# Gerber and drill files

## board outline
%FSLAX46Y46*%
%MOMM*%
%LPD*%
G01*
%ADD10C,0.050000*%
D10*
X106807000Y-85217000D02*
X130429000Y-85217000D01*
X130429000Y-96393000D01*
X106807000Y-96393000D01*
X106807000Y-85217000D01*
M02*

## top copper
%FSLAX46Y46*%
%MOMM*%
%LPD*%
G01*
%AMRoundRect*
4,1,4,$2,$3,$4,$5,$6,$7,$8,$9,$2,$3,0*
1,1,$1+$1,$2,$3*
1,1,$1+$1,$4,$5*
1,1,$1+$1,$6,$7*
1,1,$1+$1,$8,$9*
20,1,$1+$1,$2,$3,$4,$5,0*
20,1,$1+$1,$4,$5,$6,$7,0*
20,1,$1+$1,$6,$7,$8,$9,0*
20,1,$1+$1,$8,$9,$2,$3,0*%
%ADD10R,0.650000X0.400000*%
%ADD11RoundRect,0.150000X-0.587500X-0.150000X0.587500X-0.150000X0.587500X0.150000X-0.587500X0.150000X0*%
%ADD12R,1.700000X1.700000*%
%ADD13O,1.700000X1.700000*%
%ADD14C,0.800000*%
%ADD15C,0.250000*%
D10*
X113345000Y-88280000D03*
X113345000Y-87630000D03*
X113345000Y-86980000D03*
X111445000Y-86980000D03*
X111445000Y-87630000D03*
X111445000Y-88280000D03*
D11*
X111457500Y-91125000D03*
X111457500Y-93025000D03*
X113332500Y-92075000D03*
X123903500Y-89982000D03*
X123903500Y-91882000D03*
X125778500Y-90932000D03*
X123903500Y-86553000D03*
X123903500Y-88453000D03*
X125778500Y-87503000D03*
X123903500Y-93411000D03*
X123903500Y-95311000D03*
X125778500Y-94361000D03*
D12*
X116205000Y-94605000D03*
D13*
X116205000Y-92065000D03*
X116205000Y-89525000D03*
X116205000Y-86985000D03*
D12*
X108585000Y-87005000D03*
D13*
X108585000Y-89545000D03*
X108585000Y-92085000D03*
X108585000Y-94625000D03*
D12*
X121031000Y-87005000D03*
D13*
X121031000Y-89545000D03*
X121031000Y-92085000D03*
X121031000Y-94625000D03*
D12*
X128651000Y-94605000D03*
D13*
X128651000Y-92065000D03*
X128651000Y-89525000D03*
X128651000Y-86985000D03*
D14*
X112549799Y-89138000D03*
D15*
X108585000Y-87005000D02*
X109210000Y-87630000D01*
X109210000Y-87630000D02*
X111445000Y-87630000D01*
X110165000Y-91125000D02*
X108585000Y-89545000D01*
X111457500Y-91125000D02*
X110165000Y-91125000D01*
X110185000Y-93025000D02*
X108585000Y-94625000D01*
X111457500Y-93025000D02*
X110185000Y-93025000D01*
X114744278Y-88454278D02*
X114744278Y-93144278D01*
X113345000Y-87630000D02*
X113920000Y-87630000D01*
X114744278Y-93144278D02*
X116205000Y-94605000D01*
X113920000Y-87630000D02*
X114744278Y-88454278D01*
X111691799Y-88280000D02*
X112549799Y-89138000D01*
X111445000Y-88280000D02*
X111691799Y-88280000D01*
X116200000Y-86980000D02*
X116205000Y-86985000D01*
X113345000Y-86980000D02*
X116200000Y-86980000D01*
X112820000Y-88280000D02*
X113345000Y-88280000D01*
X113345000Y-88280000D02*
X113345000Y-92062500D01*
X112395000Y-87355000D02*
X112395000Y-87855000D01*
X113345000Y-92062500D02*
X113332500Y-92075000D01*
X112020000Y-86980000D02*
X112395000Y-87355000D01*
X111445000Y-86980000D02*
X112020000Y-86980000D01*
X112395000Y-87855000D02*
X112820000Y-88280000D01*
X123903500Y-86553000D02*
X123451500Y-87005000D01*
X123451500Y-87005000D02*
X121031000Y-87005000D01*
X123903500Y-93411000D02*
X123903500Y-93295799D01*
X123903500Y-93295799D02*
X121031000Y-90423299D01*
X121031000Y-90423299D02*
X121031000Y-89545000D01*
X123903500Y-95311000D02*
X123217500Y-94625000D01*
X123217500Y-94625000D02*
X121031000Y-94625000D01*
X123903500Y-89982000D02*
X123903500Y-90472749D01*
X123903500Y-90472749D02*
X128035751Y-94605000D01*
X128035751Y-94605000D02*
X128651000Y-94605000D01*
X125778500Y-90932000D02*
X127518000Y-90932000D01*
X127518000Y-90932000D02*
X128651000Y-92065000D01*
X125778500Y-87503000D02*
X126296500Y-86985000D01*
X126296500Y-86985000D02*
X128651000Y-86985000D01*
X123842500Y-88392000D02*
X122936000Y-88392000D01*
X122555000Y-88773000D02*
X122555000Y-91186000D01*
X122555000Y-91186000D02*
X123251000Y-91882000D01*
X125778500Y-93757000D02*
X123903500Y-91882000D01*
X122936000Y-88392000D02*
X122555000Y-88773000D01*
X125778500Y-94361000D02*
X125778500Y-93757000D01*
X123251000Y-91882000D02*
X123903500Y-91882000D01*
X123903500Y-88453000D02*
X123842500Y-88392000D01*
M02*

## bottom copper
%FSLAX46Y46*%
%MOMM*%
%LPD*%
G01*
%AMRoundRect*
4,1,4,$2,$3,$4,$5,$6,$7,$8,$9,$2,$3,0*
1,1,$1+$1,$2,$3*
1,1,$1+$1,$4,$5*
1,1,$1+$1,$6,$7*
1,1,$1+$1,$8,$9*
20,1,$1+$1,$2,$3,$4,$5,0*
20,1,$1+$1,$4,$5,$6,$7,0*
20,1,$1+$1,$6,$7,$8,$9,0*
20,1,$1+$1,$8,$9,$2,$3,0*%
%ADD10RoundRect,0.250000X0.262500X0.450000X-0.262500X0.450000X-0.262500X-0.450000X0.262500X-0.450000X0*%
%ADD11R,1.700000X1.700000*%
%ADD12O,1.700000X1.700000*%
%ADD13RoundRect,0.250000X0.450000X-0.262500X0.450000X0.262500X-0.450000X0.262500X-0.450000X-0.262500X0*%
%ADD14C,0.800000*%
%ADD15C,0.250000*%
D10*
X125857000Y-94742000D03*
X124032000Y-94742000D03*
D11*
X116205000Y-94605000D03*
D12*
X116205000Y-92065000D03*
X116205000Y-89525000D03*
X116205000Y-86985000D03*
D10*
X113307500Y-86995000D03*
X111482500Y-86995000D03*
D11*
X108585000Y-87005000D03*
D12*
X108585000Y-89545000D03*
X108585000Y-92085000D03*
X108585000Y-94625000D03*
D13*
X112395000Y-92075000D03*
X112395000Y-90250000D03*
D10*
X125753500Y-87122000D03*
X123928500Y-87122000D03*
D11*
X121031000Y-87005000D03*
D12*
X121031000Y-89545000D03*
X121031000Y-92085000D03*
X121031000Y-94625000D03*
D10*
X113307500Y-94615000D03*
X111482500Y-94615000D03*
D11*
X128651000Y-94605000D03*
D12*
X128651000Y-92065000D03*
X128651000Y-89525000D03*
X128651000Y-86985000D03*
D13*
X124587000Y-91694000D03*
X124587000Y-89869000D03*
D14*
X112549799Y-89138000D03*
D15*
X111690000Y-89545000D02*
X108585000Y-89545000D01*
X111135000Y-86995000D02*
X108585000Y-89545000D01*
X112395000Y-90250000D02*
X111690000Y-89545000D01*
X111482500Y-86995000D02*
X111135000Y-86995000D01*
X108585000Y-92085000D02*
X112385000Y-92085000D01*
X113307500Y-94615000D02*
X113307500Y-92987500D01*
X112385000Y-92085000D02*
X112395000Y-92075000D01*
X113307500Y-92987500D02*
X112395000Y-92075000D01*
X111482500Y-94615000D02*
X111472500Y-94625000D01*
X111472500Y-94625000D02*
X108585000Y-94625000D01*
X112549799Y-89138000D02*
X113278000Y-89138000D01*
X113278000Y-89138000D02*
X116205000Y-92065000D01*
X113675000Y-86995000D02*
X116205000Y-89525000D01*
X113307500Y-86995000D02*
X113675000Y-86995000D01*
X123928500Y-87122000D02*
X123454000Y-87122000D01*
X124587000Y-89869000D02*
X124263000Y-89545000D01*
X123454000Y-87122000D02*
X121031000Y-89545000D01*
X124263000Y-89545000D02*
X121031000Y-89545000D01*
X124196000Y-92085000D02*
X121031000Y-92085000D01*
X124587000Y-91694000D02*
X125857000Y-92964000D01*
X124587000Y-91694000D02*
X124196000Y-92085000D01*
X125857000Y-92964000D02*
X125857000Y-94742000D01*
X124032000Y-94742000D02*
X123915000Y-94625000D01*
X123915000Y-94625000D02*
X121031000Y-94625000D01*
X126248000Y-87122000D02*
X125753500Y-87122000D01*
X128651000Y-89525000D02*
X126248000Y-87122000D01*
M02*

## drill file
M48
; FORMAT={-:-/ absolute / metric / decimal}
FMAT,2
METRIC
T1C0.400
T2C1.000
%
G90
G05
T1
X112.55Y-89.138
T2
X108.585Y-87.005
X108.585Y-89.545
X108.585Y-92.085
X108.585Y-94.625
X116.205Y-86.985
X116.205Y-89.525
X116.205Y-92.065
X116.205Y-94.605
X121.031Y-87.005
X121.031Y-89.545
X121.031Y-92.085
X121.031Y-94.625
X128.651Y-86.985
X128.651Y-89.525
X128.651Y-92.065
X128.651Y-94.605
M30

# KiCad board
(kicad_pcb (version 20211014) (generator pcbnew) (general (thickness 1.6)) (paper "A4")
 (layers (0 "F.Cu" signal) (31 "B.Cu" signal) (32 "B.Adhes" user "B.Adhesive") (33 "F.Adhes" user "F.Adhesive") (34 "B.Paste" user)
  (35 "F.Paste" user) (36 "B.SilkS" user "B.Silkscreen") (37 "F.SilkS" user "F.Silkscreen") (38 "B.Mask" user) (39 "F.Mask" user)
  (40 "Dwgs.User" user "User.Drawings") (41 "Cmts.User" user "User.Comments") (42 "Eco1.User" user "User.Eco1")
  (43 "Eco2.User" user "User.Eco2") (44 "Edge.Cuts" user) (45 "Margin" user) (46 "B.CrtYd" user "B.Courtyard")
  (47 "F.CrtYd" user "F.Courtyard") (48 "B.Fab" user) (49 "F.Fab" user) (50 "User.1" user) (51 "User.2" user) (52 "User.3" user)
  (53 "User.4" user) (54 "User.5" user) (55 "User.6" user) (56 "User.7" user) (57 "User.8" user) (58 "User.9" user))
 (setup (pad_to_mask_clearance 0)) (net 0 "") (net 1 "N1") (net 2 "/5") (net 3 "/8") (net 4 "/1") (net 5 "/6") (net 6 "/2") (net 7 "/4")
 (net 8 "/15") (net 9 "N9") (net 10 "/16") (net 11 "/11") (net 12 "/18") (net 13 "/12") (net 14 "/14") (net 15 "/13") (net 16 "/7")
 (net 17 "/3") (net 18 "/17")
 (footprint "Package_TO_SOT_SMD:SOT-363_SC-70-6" (layer "F.Cu") (at 112.395 87.63 180)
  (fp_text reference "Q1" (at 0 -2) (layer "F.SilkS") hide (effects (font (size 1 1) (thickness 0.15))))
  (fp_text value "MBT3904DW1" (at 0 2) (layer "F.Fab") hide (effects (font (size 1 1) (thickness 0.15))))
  (pad "1" smd rect (at -0.95 -0.65 180) (size 0.65 0.4) (layers "F.Cu" "F.Paste" "F.Mask") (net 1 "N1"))
  (pad "2" smd rect (at -0.95 0 180) (size 0.65 0.4) (layers "F.Cu" "F.Paste" "F.Mask") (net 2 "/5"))
  (pad "3" smd rect (at -0.95 0.65 180) (size 0.65 0.4) (layers "F.Cu" "F.Paste" "F.Mask") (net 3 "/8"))
  (pad "4" smd rect (at 0.95 0.65 180) (size 0.65 0.4) (layers "F.Cu" "F.Paste" "F.Mask") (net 1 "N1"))
  (pad "5" smd rect (at 0.95 0 180) (size 0.65 0.4) (layers "F.Cu" "F.Paste" "F.Mask") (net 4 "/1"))
  (pad "6" smd rect (at 0.95 -0.65 180) (size 0.65 0.4) (layers "F.Cu" "F.Paste" "F.Mask") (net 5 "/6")))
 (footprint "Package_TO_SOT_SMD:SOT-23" (layer "F.Cu") (at 112.395 92.075)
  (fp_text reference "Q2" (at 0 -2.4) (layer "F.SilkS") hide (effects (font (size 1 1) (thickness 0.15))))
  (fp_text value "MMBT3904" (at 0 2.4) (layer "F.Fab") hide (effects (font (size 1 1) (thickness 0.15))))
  (pad "1" smd roundrect (at -0.9375 -0.95) (size 1.475 0.6) (layers "F.Cu" "F.Paste" "F.Mask") (roundrect_rratio 0.25) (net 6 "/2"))
  (pad "2" smd roundrect (at -0.9375 0.95) (size 1.475 0.6) (layers "F.Cu" "F.Paste" "F.Mask") (roundrect_rratio 0.25) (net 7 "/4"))
  (pad "3" smd roundrect (at 0.9375 0) (size 1.475 0.6) (layers "F.Cu" "F.Paste" "F.Mask") (roundrect_rratio 0.25) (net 1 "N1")))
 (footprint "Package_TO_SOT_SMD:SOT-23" (layer "F.Cu") (at 124.841 90.932)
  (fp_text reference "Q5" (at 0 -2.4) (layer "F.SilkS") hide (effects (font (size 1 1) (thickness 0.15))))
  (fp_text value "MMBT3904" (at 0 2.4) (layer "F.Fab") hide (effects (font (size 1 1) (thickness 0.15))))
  (pad "1" smd roundrect (at -0.9375 -0.95) (size 1.475 0.6) (layers "F.Cu" "F.Paste" "F.Mask") (roundrect_rratio 0.25) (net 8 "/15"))
  (pad "2" smd roundrect (at -0.9375 0.95) (size 1.475 0.6) (layers "F.Cu" "F.Paste" "F.Mask") (roundrect_rratio 0.25) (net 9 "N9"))
  (pad "3" smd roundrect (at 0.9375 0) (size 1.475 0.6) (layers "F.Cu" "F.Paste" "F.Mask") (roundrect_rratio 0.25) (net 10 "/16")))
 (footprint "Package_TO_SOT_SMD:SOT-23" (layer "F.Cu") (at 124.841 87.503)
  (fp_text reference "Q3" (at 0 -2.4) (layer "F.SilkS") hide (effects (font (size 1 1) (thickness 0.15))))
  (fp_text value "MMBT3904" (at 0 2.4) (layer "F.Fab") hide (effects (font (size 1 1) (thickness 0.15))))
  (pad "1" smd roundrect (at -0.9375 -0.95) (size 1.475 0.6) (layers "F.Cu" "F.Paste" "F.Mask") (roundrect_rratio 0.25) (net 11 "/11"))
  (pad "2" smd roundrect (at -0.9375 0.95) (size 1.475 0.6) (layers "F.Cu" "F.Paste" "F.Mask") (roundrect_rratio 0.25) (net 9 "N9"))
  (pad "3" smd roundrect (at 0.9375 0) (size 1.475 0.6) (layers "F.Cu" "F.Paste" "F.Mask") (roundrect_rratio 0.25) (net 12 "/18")))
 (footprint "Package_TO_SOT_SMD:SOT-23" (layer "F.Cu") (at 124.841 94.361)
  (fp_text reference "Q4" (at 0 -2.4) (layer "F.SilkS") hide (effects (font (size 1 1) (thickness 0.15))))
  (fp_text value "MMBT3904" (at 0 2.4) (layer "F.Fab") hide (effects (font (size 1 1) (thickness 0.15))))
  (pad "1" smd roundrect (at -0.9375 -0.95) (size 1.475 0.6) (layers "F.Cu" "F.Paste" "F.Mask") (roundrect_rratio 0.25) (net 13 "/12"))
  (pad "2" smd roundrect (at -0.9375 0.95) (size 1.475 0.6) (layers "F.Cu" "F.Paste" "F.Mask") (roundrect_rratio 0.25) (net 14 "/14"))
  (pad "3" smd roundrect (at 0.9375 0) (size 1.475 0.6) (layers "F.Cu" "F.Paste" "F.Mask") (roundrect_rratio 0.25) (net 9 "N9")))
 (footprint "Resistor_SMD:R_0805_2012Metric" (layer "B.Cu") (at 124.9445 94.742 180)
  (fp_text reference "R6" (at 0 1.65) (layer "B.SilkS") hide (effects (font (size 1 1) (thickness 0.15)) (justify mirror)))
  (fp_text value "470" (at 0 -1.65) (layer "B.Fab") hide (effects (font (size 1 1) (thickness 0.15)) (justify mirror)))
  (pad "1" smd roundrect (at -0.9125 0 180) (size 1.025 1.4) (layers "B.Cu" "B.Paste" "B.Mask") (roundrect_rratio 0.243902) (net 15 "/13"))
  (pad "2" smd roundrect (at 0.9125 0 180) (size 1.025 1.4) (layers "B.Cu" "B.Paste" "B.Mask") (roundrect_rratio 0.243902) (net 14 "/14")))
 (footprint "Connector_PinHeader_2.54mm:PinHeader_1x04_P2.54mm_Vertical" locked (layer "B.Cu") (at 116.205 94.605)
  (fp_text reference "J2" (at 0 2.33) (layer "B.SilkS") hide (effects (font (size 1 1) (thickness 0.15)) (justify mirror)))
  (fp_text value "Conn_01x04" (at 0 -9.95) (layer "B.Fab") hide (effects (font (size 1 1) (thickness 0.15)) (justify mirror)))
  (pad "1" thru_hole rect locked (at 0 0) (size 1.7 1.7) (drill 1) (layers *.Cu *.Mask) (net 2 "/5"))
  (pad "2" thru_hole oval locked (at 0 -2.54) (size 1.7 1.7) (drill 1) (layers *.Cu *.Mask) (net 5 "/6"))
  (pad "3" thru_hole oval locked (at 0 -5.08) (size 1.7 1.7) (drill 1) (layers *.Cu *.Mask) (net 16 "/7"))
  (pad "4" thru_hole oval locked (at 0 -7.62) (size 1.7 1.7) (drill 1) (layers *.Cu *.Mask) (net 3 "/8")))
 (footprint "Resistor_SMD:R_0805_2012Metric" (layer "B.Cu") (at 112.395 86.995 180)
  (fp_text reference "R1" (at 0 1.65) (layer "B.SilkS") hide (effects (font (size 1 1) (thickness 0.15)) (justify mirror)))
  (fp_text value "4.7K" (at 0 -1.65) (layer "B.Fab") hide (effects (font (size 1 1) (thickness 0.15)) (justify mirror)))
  (pad "1" smd roundrect (at -0.9125 0 180) (size 1.025 1.4) (layers "B.Cu" "B.Paste" "B.Mask") (roundrect_rratio 0.243902) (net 16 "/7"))
  (pad "2" smd roundrect (at 0.9125 0 180) (size 1.025 1.4) (layers "B.Cu" "B.Paste" "B.Mask") (roundrect_rratio 0.243902) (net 6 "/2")))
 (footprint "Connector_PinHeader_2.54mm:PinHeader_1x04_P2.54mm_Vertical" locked (layer "B.Cu") (at 108.585 87.005 180)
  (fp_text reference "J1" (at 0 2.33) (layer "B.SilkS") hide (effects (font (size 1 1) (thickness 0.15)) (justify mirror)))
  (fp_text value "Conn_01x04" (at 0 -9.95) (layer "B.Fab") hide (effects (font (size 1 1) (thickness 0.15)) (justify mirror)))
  (pad "1" thru_hole rect locked (at 0 0 180) (size 1.7 1.7) (drill 1) (layers *.Cu *.Mask) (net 4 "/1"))
  (pad "2" thru_hole oval locked (at 0 -2.54 180) (size 1.7 1.7) (drill 1) (layers *.Cu *.Mask) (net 6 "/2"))
  (pad "3" thru_hole oval locked (at 0 -5.08 180) (size 1.7 1.7) (drill 1) (layers *.Cu *.Mask) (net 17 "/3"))
  (pad "4" thru_hole oval locked (at 0 -7.62 180) (size 1.7 1.7) (drill 1) (layers *.Cu *.Mask) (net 7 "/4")))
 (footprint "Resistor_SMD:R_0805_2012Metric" (layer "B.Cu") (at 112.395 91.1625 90)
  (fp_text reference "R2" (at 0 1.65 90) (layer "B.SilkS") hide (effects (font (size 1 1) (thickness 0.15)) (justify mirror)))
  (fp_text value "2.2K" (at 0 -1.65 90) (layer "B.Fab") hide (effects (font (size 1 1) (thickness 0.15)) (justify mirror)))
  (pad "1" smd roundrect (at -0.9125 0 90) (size 1.025 1.4) (layers "B.Cu" "B.Paste" "B.Mask") (roundrect_rratio 0.243902) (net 17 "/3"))
  (pad "2" smd roundrect (at 0.9125 0 90) (size 1.025 1.4) (layers "B.Cu" "B.Paste" "B.Mask") (roundrect_rratio 0.243902) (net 6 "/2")))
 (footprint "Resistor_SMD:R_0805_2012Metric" (layer "B.Cu") (at 124.841 87.122 180)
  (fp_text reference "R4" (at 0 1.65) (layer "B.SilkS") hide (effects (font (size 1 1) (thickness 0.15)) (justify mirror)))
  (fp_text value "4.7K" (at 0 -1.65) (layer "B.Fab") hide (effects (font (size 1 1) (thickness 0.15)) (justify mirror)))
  (pad "1" smd roundrect (at -0.9125 0 180) (size 1.025 1.4) (layers "B.Cu" "B.Paste" "B.Mask") (roundrect_rratio 0.243902) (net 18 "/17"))
  (pad "2" smd roundrect (at 0.9125 0 180) (size 1.025 1.4) (layers "B.Cu" "B.Paste" "B.Mask") (roundrect_rratio 0.243902) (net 13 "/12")))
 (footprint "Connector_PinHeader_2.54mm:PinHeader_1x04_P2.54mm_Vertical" (layer "B.Cu") (at 121.031 87.005 180)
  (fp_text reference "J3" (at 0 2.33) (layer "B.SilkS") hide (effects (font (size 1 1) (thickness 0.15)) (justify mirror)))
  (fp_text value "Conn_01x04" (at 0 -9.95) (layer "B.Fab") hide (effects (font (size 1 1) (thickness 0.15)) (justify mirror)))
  (pad "1" thru_hole rect locked (at 0 0 180) (size 1.7 1.7) (drill 1) (layers *.Cu *.Mask) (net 11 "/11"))
  (pad "2" thru_hole oval locked (at 0 -2.54 180) (size 1.7 1.7) (drill 1) (layers *.Cu *.Mask) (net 13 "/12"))
  (pad "3" thru_hole oval locked (at 0 -5.08 180) (size 1.7 1.7) (drill 1) (layers *.Cu *.Mask) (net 15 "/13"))
  (pad "4" thru_hole oval locked (at 0 -7.62 180) (size 1.7 1.7) (drill 1) (layers *.Cu *.Mask) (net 14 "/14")))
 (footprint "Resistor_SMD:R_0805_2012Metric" (layer "B.Cu") (at 112.395 94.615 180)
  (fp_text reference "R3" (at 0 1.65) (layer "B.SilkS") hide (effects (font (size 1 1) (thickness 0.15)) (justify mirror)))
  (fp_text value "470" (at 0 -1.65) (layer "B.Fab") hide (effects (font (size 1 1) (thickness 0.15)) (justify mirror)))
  (pad "1" smd roundrect (at -0.9125 0 180) (size 1.025 1.4) (layers "B.Cu" "B.Paste" "B.Mask") (roundrect_rratio 0.243902) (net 17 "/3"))
  (pad "2" smd roundrect (at 0.9125 0 180) (size 1.025 1.4) (layers "B.Cu" "B.Paste" "B.Mask") (roundrect_rratio 0.243902) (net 7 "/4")))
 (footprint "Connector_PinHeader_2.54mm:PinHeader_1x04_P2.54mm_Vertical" (layer "B.Cu") (at 128.651 94.605)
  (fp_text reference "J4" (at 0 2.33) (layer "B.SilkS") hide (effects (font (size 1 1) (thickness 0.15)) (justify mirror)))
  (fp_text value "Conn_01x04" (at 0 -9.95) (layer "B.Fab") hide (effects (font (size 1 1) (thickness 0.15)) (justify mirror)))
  (pad "1" thru_hole rect locked (at 0 0) (size 1.7 1.7) (drill 1) (layers *.Cu *.Mask) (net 8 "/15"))
  (pad "2" thru_hole oval locked (at 0 -2.54) (size 1.7 1.7) (drill 1) (layers *.Cu *.Mask) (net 10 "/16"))
  (pad "3" thru_hole oval locked (at 0 -5.08) (size 1.7 1.7) (drill 1) (layers *.Cu *.Mask) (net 18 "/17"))
  (pad "4" thru_hole oval locked (at 0 -7.62) (size 1.7 1.7) (drill 1) (layers *.Cu *.Mask) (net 12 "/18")))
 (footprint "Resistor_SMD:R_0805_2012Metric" (layer "B.Cu") (at 124.587 90.7815 90)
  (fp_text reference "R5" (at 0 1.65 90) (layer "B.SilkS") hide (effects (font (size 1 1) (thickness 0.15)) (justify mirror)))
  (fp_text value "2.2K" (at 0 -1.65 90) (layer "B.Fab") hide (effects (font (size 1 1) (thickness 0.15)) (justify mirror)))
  (pad "1" smd roundrect (at -0.9125 0 90) (size 1.025 1.4) (layers "B.Cu" "B.Paste" "B.Mask") (roundrect_rratio 0.243902) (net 15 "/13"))
  (pad "2" smd roundrect (at 0.9125 0 90) (size 1.025 1.4) (layers "B.Cu" "B.Paste" "B.Mask") (roundrect_rratio 0.243902) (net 13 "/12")))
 (gr_rect (start 106.807 85.217) (end 130.429 96.393) (layer "Edge.Cuts") (width 0.05) (fill none))
 (segment (start 108.585 87.005) (end 109.21 87.63) (width 0.25) (layer "F.Cu") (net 4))
 (segment (start 109.21 87.63) (end 111.445 87.63) (width 0.25) (layer "F.Cu") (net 4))
 (segment (start 110.165 91.125) (end 108.585 89.545) (width 0.25) (layer "F.Cu") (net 6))
 (segment (start 111.4575 91.125) (end 110.165 91.125) (width 0.25) (layer "F.Cu") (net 6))
 (segment (start 111.69 89.545) (end 108.585 89.545) (width 0.25) (layer "B.Cu") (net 6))
 (segment (start 111.135 86.995) (end 108.585 89.545) (width 0.25) (layer "B.Cu") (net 6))
 (segment (start 112.395 90.25) (end 111.69 89.545) (width 0.25) (layer "B.Cu") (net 6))
 (segment (start 111.4825 86.995) (end 111.135 86.995) (width 0.25) (layer "B.Cu") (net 6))
 (segment (start 108.585 92.085) (end 112.385 92.085) (width 0.25) (layer "B.Cu") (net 17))
 (segment (start 113.3075 94.615) (end 113.3075 92.9875) (width 0.25) (layer "B.Cu") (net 17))
 (segment (start 112.385 92.085) (end 112.395 92.075) (width 0.25) (layer "B.Cu") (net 17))
 (segment (start 113.3075 92.9875) (end 112.395 92.075) (width 0.25) (layer "B.Cu") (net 17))
 (segment (start 110.185 93.025) (end 108.585 94.625) (width 0.25) (layer "F.Cu") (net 7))
 (segment (start 111.4575 93.025) (end 110.185 93.025) (width 0.25) (layer "F.Cu") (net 7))
 (segment (start 111.4825 94.615) (end 111.4725 94.625) (width 0.25) (layer "B.Cu") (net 7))
 (segment (start 111.4725 94.625) (end 108.585 94.625) (width 0.25) (layer "B.Cu") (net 7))
 (segment (start 114.744278 88.454278) (end 114.744278 93.144278) (width 0.25) (layer "F.Cu") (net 2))
 (segment (start 113.345 87.63) (end 113.92 87.63) (width 0.25) (layer "F.Cu") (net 2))
 (segment (start 114.744278 93.144278) (end 116.205 94.605) (width 0.25) (layer "F.Cu") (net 2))
 (segment (start 113.92 87.63) (end 114.744278 88.454278) (width 0.25) (layer "F.Cu") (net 2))
 (segment (start 111.691799 88.28) (end 112.549799 89.138) (width 0.25) (layer "F.Cu") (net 5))
 (segment (start 111.445 88.28) (end 111.691799 88.28) (width 0.25) (layer "F.Cu") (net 5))
 (via (at 112.549799 89.138) (size 0.8) (drill 0.4) (layers "F.Cu" "B.Cu") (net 5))
 (segment (start 112.549799 89.138) (end 113.278 89.138) (width 0.25) (layer "B.Cu") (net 5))
 (segment (start 113.278 89.138) (end 116.205 92.065) (width 0.25) (layer "B.Cu") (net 5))
 (segment (start 113.675 86.995) (end 116.205 89.525) (width 0.25) (layer "B.Cu") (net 16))
 (segment (start 113.3075 86.995) (end 113.675 86.995) (width 0.25) (layer "B.Cu") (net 16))
 (segment (start 116.2 86.98) (end 116.205 86.985) (width 0.25) (layer "F.Cu") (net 3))
 (segment (start 113.345 86.98) (end 116.2 86.98) (width 0.25) (layer "F.Cu") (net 3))
 (segment (start 112.82 88.28) (end 113.345 88.28) (width 0.25) (layer "F.Cu") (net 1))
 (segment (start 113.345 88.28) (end 113.345 92.0625) (width 0.25) (layer "F.Cu") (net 1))
 (segment (start 112.395 87.355) (end 112.395 87.855) (width 0.25) (layer "F.Cu") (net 1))
 (segment (start 113.345 92.0625) (end 113.3325 92.075) (width 0.25) (layer "F.Cu") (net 1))
 (segment (start 112.02 86.98) (end 112.395 87.355) (width 0.25) (layer "F.Cu") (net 1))
 (segment (start 111.445 86.98) (end 112.02 86.98) (width 0.25) (layer "F.Cu") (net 1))
 (segment (start 112.395 87.855) (end 112.82 88.28) (width 0.25) (layer "F.Cu") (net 1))
 (segment (start 123.9035 86.553) (end 123.4515 87.005) (width 0.25) (layer "F.Cu") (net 11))
 (segment (start 123.4515 87.005) (end 121.031 87.005) (width 0.25) (layer "F.Cu") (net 11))
 (segment (start 123.9035 93.411) (end 123.9035 93.295799) (width 0.25) (layer "F.Cu") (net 13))
 (segment (start 123.9035 93.295799) (end 121.031 90.423299) (width 0.25) (layer "F.Cu") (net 13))
 (segment (start 121.031 90.423299) (end 121.031 89.545) (width 0.25) (layer "F.Cu") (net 13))
 (segment (start 123.9285 87.122) (end 123.454 87.122) (width 0.25) (layer "B.Cu") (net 13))
 (segment (start 124.587 89.869) (end 124.263 89.545) (width 0.25) (layer "B.Cu") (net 13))
 (segment (start 123.454 87.122) (end 121.031 89.545) (width 0.25) (layer "B.Cu") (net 13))
 (segment (start 124.263 89.545) (end 121.031 89.545) (width 0.25) (layer "B.Cu") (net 13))
 (segment (start 124.196 92.085) (end 121.031 92.085) (width 0.25) (layer "B.Cu") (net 15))
 (segment (start 124.587 91.694) (end 125.857 92.964) (width 0.25) (layer "B.Cu") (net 15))
 (segment (start 124.587 91.694) (end 124.196 92.085) (width 0.25) (layer "B.Cu") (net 15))
 (segment (start 125.857 92.964) (end 125.857 94.742) (width 0.25) (layer "B.Cu") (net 15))
 (segment (start 123.9035 95.311) (end 123.2175 94.625) (width 0.25) (layer "F.Cu") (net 14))
 (segment (start 123.2175 94.625) (end 121.031 94.625) (width 0.25) (layer "F.Cu") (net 14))
 (segment (start 124.032 94.742) (end 123.915 94.625) (width 0.25) (layer "B.Cu") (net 14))
 (segment (start 123.915 94.625) (end 121.031 94.625) (width 0.25) (layer "B.Cu") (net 14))
 (segment (start 123.9035 89.982) (end 123.9035 90.472749) (width 0.25) (layer "F.Cu") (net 8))
 (segment (start 123.9035 90.472749) (end 128.035751 94.605) (width 0.25) (layer "F.Cu") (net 8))
 (segment (start 128.035751 94.605) (end 128.651 94.605) (width 0.25) (layer "F.Cu") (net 8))
 (segment (start 125.7785 90.932) (end 127.518 90.932) (width 0.25) (layer "F.Cu") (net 10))
 (segment (start 127.518 90.932) (end 128.651 92.065) (width 0.25) (layer "F.Cu") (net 10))
 (segment (start 126.248 87.122) (end 125.7535 87.122) (width 0.25) (layer "B.Cu") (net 18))
 (segment (start 128.651 89.525) (end 126.248 87.122) (width 0.25) (layer "B.Cu") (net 18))
 (segment (start 125.7785 87.503) (end 126.2965 86.985) (width 0.25) (layer "F.Cu") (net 12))
 (segment (start 126.2965 86.985) (end 128.651 86.985) (width 0.25) (layer "F.Cu") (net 12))
 (segment (start 123.8425 88.392) (end 122.936 88.392) (width 0.25) (layer "F.Cu") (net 9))
 (segment (start 122.555 88.773) (end 122.555 91.186) (width 0.25) (layer "F.Cu") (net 9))
 (segment (start 122.555 91.186) (end 123.251 91.882) (width 0.25) (layer "F.Cu") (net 9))
 (segment (start 125.7785 93.757) (end 123.9035 91.882) (width 0.25) (layer "F.Cu") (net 9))
 (segment (start 122.936 88.392) (end 122.555 88.773) (width 0.25) (layer "F.Cu") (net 9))
 (segment (start 125.7785 94.361) (end 125.7785 93.757) (width 0.25) (layer "F.Cu") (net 9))
 (segment (start 123.251 91.882) (end 123.9035 91.882) (width 0.25) (layer "F.Cu") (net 9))
 (segment (start 123.9035 88.453) (end 123.8425 88.392) (width 0.25) (layer "F.Cu") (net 9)))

